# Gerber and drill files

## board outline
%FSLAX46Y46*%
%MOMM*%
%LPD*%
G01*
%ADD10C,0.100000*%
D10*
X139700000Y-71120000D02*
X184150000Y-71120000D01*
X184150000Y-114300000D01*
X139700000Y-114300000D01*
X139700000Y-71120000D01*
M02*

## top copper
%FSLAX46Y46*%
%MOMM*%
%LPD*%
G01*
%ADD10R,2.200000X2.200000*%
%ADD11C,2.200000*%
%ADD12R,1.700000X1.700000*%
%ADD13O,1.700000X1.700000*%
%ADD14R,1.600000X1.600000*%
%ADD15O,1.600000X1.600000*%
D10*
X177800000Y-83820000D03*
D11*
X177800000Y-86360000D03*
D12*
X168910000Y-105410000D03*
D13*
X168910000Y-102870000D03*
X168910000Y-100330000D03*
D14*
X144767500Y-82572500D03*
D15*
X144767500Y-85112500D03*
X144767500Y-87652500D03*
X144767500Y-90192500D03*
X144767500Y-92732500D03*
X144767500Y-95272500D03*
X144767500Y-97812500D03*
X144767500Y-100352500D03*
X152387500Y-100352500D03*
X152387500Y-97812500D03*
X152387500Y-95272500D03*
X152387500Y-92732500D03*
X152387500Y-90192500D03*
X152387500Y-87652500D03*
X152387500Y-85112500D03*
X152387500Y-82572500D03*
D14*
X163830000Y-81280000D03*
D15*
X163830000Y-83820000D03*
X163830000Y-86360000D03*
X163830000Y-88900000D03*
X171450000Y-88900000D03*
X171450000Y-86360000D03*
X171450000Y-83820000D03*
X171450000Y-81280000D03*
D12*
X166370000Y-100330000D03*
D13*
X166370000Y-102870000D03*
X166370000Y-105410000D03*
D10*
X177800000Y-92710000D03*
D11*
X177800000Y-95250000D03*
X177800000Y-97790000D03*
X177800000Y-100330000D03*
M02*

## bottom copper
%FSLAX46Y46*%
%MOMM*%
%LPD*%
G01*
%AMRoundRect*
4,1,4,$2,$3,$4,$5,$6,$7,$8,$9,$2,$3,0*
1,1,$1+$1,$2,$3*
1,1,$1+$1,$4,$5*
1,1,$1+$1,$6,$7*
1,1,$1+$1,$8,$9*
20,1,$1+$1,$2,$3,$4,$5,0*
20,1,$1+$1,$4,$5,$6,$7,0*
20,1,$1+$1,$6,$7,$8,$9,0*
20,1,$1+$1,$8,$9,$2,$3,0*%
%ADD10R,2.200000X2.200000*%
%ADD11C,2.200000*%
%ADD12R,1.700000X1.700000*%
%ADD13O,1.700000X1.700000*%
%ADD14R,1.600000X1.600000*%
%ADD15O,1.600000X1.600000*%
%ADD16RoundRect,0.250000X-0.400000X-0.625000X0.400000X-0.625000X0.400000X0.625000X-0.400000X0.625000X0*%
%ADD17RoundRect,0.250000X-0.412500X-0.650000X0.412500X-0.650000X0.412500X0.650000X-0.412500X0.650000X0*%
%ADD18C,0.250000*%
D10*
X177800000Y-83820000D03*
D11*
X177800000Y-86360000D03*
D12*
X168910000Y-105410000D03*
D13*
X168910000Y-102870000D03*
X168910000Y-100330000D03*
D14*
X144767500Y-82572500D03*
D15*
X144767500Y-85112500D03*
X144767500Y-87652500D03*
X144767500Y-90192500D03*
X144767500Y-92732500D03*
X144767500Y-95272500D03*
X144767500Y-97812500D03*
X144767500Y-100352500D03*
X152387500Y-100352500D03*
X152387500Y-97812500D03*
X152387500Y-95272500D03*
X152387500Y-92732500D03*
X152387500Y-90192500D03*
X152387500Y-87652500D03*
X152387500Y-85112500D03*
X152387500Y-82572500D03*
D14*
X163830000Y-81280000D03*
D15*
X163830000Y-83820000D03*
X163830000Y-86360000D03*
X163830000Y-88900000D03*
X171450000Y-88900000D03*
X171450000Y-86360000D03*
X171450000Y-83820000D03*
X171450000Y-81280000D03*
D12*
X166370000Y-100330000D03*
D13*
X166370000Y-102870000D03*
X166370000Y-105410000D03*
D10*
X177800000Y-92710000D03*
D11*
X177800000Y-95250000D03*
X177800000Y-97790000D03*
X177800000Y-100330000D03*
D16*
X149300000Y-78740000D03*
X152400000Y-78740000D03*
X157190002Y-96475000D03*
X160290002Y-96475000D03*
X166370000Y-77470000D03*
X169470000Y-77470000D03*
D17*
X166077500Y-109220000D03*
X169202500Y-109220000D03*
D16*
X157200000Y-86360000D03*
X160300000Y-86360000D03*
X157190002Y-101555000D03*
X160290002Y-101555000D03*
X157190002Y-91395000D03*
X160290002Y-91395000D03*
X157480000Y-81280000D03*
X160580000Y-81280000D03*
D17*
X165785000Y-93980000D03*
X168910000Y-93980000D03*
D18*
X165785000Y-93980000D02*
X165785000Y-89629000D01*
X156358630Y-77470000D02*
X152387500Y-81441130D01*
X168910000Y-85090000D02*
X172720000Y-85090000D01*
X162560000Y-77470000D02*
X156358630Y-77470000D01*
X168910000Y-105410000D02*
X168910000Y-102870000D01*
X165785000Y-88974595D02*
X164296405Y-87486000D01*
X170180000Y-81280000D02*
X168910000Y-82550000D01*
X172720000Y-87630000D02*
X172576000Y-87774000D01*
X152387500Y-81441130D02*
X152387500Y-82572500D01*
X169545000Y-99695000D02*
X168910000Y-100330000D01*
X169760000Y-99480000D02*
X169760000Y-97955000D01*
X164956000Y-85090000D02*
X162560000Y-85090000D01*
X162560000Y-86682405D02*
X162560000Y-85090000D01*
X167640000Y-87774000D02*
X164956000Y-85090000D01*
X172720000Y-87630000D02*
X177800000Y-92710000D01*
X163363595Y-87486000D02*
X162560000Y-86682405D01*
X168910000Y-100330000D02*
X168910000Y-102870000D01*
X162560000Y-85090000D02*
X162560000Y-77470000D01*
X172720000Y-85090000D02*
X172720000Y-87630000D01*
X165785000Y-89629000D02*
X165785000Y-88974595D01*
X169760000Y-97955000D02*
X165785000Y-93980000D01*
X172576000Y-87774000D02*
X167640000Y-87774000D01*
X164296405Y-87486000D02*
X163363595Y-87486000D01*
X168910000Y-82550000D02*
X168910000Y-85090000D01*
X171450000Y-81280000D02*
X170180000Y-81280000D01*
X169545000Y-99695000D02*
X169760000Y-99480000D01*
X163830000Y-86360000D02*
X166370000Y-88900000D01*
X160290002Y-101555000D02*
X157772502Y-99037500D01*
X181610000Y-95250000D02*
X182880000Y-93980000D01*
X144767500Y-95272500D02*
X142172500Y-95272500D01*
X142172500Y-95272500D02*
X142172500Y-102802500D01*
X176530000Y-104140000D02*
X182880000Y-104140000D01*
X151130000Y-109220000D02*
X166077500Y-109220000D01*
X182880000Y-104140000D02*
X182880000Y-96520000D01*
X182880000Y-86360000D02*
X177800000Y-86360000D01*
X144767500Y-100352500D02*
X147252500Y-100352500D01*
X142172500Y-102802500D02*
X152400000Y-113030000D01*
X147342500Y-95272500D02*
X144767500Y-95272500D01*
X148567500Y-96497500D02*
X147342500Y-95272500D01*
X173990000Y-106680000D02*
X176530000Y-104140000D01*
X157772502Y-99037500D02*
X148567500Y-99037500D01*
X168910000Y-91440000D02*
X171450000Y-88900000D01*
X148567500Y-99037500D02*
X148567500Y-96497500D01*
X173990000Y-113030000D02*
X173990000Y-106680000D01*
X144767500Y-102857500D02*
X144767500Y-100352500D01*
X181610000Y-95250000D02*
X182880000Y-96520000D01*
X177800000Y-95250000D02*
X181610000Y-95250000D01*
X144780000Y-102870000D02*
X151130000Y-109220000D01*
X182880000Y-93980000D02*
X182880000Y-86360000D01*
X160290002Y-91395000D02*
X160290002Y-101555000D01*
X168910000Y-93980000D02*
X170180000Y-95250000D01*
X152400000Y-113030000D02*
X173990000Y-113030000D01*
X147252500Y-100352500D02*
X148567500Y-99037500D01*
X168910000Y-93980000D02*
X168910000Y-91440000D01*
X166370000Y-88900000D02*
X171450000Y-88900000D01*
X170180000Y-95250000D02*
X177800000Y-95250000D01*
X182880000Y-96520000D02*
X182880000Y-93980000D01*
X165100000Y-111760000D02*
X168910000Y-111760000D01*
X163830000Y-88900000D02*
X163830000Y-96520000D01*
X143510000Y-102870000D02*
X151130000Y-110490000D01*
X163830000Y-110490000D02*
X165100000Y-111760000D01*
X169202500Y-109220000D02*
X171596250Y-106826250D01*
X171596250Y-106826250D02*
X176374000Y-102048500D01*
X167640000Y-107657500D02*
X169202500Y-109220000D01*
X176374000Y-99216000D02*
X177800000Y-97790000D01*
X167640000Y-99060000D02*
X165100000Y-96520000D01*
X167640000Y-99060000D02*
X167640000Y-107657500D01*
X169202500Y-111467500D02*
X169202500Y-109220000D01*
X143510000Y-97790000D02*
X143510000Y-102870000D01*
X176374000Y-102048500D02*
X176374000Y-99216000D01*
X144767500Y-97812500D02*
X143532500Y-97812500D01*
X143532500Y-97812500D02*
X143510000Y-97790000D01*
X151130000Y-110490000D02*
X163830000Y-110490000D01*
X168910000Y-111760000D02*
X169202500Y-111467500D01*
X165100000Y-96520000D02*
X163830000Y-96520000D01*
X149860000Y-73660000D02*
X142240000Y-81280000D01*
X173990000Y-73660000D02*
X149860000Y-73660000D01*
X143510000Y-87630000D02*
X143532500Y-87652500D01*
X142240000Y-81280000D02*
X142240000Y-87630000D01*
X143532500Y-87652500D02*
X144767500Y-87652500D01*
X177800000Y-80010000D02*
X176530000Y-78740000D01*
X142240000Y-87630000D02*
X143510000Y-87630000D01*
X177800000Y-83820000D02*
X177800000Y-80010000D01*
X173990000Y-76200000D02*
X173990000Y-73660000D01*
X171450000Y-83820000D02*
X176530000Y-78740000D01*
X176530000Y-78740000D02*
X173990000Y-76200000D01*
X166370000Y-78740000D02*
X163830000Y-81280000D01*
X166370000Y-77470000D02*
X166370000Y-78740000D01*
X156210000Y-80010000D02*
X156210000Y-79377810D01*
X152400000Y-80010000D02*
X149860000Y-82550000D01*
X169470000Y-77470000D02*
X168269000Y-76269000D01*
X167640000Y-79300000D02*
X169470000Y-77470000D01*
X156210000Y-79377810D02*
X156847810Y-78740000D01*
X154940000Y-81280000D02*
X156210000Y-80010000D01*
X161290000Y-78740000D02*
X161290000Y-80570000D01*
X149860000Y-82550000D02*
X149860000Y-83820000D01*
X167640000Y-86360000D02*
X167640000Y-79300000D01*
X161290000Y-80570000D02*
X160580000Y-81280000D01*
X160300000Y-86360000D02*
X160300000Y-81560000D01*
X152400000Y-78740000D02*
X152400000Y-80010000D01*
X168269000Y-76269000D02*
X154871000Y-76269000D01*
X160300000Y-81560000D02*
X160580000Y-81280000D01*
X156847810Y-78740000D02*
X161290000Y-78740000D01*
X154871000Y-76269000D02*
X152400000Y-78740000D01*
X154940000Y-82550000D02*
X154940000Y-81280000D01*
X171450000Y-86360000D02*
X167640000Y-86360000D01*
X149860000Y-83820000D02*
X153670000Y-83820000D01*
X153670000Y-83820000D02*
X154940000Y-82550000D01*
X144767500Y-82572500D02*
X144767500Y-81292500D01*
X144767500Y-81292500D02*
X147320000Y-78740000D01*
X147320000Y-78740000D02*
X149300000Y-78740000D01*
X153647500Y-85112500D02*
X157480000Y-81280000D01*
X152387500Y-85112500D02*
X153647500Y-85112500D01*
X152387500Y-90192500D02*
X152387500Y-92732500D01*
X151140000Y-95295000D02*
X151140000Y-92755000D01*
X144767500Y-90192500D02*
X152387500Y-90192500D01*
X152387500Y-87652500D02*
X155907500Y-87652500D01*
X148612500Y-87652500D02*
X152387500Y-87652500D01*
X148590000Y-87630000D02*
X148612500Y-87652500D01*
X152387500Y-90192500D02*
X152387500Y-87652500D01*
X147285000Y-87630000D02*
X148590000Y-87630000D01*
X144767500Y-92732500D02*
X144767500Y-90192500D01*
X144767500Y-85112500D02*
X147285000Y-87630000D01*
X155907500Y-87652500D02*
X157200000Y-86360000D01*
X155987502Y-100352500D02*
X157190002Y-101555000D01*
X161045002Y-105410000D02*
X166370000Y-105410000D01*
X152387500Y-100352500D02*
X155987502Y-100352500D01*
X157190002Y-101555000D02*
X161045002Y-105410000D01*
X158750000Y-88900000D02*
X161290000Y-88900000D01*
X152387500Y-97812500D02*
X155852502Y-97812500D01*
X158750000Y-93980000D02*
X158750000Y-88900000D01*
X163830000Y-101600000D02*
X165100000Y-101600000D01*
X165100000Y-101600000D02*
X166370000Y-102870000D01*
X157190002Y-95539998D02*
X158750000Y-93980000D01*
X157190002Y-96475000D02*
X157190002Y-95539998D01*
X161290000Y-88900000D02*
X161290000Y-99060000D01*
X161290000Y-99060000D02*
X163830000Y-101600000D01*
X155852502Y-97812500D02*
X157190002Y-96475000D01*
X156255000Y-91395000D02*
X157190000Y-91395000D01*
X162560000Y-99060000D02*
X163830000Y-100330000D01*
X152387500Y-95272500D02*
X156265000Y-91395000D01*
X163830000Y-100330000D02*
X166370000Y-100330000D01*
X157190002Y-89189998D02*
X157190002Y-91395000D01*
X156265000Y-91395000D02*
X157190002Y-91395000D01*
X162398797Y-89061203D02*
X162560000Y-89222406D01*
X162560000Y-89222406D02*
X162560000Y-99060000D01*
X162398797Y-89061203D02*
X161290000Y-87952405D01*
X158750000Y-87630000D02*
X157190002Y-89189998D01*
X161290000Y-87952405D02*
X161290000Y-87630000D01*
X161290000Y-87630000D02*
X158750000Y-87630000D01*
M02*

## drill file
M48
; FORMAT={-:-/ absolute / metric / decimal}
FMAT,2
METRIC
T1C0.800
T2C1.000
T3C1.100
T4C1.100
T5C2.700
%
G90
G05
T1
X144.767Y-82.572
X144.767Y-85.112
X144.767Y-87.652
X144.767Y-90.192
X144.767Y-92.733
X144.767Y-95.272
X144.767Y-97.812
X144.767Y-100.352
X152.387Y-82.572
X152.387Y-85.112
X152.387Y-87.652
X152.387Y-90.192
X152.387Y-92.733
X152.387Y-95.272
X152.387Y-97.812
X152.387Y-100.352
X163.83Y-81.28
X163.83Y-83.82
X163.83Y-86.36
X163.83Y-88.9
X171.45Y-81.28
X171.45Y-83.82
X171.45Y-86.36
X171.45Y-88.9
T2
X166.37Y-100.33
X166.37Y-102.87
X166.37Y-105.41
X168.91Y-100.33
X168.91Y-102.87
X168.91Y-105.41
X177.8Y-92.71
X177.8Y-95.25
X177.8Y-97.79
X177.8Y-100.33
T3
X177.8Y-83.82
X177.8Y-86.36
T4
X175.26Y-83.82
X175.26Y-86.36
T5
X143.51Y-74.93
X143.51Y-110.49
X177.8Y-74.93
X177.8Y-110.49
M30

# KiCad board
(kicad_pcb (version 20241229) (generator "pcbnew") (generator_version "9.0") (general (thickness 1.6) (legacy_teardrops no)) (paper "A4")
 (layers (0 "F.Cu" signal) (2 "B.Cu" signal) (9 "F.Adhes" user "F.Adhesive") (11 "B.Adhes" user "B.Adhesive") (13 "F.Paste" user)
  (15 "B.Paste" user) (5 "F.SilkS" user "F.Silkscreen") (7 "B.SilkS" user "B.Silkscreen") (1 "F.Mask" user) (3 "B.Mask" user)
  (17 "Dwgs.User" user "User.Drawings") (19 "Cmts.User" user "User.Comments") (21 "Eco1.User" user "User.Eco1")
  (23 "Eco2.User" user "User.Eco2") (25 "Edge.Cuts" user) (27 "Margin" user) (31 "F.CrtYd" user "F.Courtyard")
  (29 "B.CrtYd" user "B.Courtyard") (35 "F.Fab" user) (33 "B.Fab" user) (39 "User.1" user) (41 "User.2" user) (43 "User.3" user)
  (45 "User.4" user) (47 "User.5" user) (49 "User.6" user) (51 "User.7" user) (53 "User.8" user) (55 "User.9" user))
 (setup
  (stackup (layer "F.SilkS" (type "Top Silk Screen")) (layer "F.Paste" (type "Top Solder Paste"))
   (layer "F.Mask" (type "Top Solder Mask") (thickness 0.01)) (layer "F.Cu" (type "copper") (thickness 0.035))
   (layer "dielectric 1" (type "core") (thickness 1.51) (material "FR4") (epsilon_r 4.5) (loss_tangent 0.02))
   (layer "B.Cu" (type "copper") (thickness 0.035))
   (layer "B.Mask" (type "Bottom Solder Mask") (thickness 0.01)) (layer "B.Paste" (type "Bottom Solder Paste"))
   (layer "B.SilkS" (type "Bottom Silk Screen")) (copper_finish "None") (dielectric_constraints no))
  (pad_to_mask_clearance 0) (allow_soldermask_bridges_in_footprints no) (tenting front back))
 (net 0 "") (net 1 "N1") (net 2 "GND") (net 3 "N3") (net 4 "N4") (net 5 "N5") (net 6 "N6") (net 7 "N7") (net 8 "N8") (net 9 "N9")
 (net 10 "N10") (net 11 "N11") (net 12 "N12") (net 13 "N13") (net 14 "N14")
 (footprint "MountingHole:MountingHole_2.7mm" (layer "F.Cu") (at 177.8 74.93)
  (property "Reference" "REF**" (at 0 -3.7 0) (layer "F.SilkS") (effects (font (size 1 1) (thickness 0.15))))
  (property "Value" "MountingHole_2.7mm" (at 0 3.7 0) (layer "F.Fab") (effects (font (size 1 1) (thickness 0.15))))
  (pad "" np_thru_hole circle (at 0 0) (size 2.7 2.7) (drill 2.7) (layers "*.Cu" "*.Mask")))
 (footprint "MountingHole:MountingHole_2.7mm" (layer "F.Cu") (at 177.8 110.49)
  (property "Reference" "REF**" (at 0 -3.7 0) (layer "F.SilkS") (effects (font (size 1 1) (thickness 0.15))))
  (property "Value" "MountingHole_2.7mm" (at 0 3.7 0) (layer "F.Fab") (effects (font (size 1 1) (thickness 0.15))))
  (pad "" np_thru_hole circle (at 0 0) (size 2.7 2.7) (drill 2.7) (layers "*.Cu" "*.Mask")))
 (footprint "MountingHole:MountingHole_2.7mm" (layer "F.Cu") (at 143.51 110.49)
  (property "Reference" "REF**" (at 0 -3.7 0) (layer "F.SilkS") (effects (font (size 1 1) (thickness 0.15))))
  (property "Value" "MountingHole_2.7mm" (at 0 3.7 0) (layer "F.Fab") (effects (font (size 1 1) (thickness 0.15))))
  (pad "" np_thru_hole circle (at 0 0) (size 2.7 2.7) (drill 2.7) (layers "*.Cu" "*.Mask")))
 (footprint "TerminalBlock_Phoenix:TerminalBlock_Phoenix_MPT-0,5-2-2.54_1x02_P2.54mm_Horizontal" (layer "F.Cu") (at 177.8 83.82 -90)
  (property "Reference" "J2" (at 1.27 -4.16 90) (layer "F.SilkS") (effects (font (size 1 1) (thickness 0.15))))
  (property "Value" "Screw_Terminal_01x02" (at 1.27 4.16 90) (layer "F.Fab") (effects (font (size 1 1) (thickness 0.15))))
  (pad "" np_thru_hole circle (at 0 2.54 270) (size 1.1 1.1) (drill 1.1) (layers "*.Cu" "*.Mask"))
  (pad "" np_thru_hole circle (at 2.54 2.54 270) (size 1.1 1.1) (drill 1.1) (layers "*.Cu" "*.Mask"))
  (pad "1" thru_hole rect (at 0 0 270) (size 2.2 2.2) (drill 1.1) (layers "*.Cu" "*.Mask") (remove_unused_layers no) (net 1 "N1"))
  (pad "2" thru_hole circle (at 2.54 0 270) (size 2.2 2.2) (drill 1.1) (layers "*.Cu" "*.Mask") (remove_unused_layers no) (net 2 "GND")))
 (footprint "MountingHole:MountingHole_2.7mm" (layer "F.Cu") (at 143.51 74.93)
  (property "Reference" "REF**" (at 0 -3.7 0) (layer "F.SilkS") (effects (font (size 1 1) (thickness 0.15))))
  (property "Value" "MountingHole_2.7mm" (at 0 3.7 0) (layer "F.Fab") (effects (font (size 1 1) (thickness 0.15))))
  (pad "" np_thru_hole circle (at 0 0) (size 2.7 2.7) (drill 2.7) (layers "*.Cu" "*.Mask")))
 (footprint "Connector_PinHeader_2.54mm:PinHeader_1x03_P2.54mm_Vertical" (layer "F.Cu") (at 168.91 105.41 180)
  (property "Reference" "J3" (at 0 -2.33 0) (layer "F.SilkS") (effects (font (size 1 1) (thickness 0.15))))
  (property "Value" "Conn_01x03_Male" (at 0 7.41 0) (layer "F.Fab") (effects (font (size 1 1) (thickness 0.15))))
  (pad "1" thru_hole rect (at 0 0 180) (size 1.7 1.7) (drill 1) (layers "*.Cu" "*.Mask") (remove_unused_layers no) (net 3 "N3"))
  (pad "2" thru_hole oval (at 0 2.54 180) (size 1.7 1.7) (drill 1) (layers "*.Cu" "*.Mask") (remove_unused_layers no) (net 3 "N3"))
  (pad "3" thru_hole oval (at 0 5.08 180) (size 1.7 1.7) (drill 1) (layers "*.Cu" "*.Mask") (remove_unused_layers no) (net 3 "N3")))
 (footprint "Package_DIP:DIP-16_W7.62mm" (layer "F.Cu") (at 144.7675 82.5725)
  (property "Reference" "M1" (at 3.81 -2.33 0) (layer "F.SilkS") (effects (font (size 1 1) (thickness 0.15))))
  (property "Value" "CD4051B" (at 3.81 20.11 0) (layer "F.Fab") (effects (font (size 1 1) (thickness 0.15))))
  (pad "1" thru_hole rect (at 0 0) (size 1.6 1.6) (drill 0.8) (layers "*.Cu" "*.Mask") (remove_unused_layers no) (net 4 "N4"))
  (pad "2" thru_hole oval (at 0 2.54) (size 1.6 1.6) (drill 0.8) (layers "*.Cu" "*.Mask") (remove_unused_layers no) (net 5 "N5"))
  (pad "3" thru_hole oval (at 0 5.08) (size 1.6 1.6) (drill 0.8) (layers "*.Cu" "*.Mask") (remove_unused_layers no) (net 1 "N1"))
  (pad "4" thru_hole oval (at 0 7.62) (size 1.6 1.6) (drill 0.8) (layers "*.Cu" "*.Mask") (remove_unused_layers no) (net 5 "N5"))
  (pad "5" thru_hole oval (at 0 10.16) (size 1.6 1.6) (drill 0.8) (layers "*.Cu" "*.Mask") (remove_unused_layers no) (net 5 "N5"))
  (pad "6" thru_hole oval (at 0 12.7) (size 1.6 1.6) (drill 0.8) (layers "*.Cu" "*.Mask") (remove_unused_layers no) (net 2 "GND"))
  (pad "7" thru_hole oval (at 0 15.24) (size 1.6 1.6) (drill 0.8) (layers "*.Cu" "*.Mask") (remove_unused_layers no) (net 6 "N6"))
  (pad "8" thru_hole oval (at 0 17.78) (size 1.6 1.6) (drill 0.8) (layers "*.Cu" "*.Mask") (remove_unused_layers no) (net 2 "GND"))
  (pad "9" thru_hole oval (at 7.62 17.78) (size 1.6 1.6) (drill 0.8) (layers "*.Cu" "*.Mask") (remove_unused_layers no) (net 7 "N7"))
  (pad "10" thru_hole oval (at 7.62 15.24) (size 1.6 1.6) (drill 0.8) (layers "*.Cu" "*.Mask") (remove_unused_layers no) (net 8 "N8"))
  (pad "11" thru_hole oval (at 7.62 12.7) (size 1.6 1.6) (drill 0.8) (layers "*.Cu" "*.Mask") (remove_unused_layers no) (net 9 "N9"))
  (pad "12" thru_hole oval (at 7.62 10.16) (size 1.6 1.6) (drill 0.8) (layers "*.Cu" "*.Mask") (remove_unused_layers no) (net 5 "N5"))
  (pad "13" thru_hole oval (at 7.62 7.62) (size 1.6 1.6) (drill 0.8) (layers "*.Cu" "*.Mask") (remove_unused_layers no) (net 5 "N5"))
  (pad "14" thru_hole oval (at 7.62 5.08) (size 1.6 1.6) (drill 0.8) (layers "*.Cu" "*.Mask") (remove_unused_layers no) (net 5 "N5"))
  (pad "15" thru_hole oval (at 7.62 2.54) (size 1.6 1.6) (drill 0.8) (layers "*.Cu" "*.Mask") (remove_unused_layers no) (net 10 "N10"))
  (pad "16" thru_hole oval (at 7.62 0) (size 1.6 1.6) (drill 0.8) (layers "*.Cu" "*.Mask") (remove_unused_layers no) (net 3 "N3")))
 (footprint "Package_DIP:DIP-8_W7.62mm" (layer "F.Cu") (at 163.83 81.28)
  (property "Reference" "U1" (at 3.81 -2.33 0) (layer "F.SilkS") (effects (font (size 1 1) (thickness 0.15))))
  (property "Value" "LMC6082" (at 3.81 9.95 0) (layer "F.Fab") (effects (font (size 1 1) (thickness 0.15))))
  (pad "1" thru_hole rect (at 0 0) (size 1.6 1.6) (drill 0.8) (layers "*.Cu" "*.Mask") (remove_unused_layers no) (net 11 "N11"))
  (pad "2" thru_hole oval (at 0 2.54) (size 1.6 1.6) (drill 0.8) (layers "*.Cu" "*.Mask") (remove_unused_layers no) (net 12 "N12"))
  (pad "3" thru_hole oval (at 0 5.08) (size 1.6 1.6) (drill 0.8) (layers "*.Cu" "*.Mask") (remove_unused_layers no) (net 2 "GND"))
  (pad "4" thru_hole oval (at 0 7.62) (size 1.6 1.6) (drill 0.8) (layers "*.Cu" "*.Mask") (remove_unused_layers no) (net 6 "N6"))
  (pad "5" thru_hole oval (at 7.62 7.62) (size 1.6 1.6) (drill 0.8) (layers "*.Cu" "*.Mask") (remove_unused_layers no) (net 2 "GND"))
  (pad "6" thru_hole oval (at 7.62 5.08) (size 1.6 1.6) (drill 0.8) (layers "*.Cu" "*.Mask") (remove_unused_layers no) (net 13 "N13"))
  (pad "7" thru_hole oval (at 7.62 2.54) (size 1.6 1.6) (drill 0.8) (layers "*.Cu" "*.Mask") (remove_unused_layers no) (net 1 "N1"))
  (pad "8" thru_hole oval (at 7.62 0) (size 1.6 1.6) (drill 0.8) (layers "*.Cu" "*.Mask") (remove_unused_layers no) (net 3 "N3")))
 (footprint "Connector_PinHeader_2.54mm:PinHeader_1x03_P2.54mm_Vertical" (layer "F.Cu") (at 166.37 100.33)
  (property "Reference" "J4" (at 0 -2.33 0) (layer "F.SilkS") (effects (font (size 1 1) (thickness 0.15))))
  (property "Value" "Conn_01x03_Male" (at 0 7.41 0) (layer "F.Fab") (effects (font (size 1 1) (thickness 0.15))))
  (pad "1" thru_hole rect (at 0 0) (size 1.7 1.7) (drill 1) (layers "*.Cu" "*.Mask") (remove_unused_layers no) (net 9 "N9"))
  (pad "2" thru_hole oval (at 0 2.54) (size 1.7 1.7) (drill 1) (layers "*.Cu" "*.Mask") (remove_unused_layers no) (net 8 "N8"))
  (pad "3" thru_hole oval (at 0 5.08) (size 1.7 1.7) (drill 1) (layers "*.Cu" "*.Mask") (remove_unused_layers no) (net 7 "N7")))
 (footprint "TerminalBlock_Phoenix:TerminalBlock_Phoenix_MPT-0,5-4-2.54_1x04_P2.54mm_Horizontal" (layer "F.Cu") (at 177.8 92.71 -90)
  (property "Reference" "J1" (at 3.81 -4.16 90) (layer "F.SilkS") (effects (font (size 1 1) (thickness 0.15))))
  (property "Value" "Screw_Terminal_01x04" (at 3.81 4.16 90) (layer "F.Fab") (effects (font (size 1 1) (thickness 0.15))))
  (pad "1" thru_hole rect (at 0 0 270) (size 2.2 2.2) (drill 1) (layers "*.Cu" "*.Mask") (remove_unused_layers no) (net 3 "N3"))
  (pad "2" thru_hole circle (at 2.54 0 270) (size 2.2 2.2) (drill 1) (layers "*.Cu" "*.Mask") (remove_unused_layers no) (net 2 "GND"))
  (pad "3" thru_hole circle (at 5.08 0 270) (size 2.2 2.2) (drill 1) (layers "*.Cu" "*.Mask") (remove_unused_layers no) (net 6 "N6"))
  (pad "4" thru_hole circle (at 7.62 0 270) (size 2.2 2.2) (drill 1) (layers "*.Cu" "*.Mask") (remove_unused_layers no) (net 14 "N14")))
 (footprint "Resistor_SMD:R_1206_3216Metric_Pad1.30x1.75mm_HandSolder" (layer "B.Cu") (at 150.85 78.74)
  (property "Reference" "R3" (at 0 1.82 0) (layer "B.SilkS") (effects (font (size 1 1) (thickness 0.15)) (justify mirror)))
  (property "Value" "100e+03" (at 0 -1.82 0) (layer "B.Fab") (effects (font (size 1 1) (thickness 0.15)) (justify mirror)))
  (pad "1" smd roundrect (at -1.55 0) (size 1.3 1.75) (layers "B.Cu" "B.Mask" "B.Paste") (roundrect_rratio 0.1923076923) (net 4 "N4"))
  (pad "2" smd roundrect (at 1.55 0) (size 1.3 1.75) (layers "B.Cu" "B.Mask" "B.Paste") (roundrect_rratio 0.1923076923) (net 13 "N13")))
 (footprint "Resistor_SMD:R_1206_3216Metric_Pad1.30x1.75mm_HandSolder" (layer "B.Cu") (at 158.740002 96.475)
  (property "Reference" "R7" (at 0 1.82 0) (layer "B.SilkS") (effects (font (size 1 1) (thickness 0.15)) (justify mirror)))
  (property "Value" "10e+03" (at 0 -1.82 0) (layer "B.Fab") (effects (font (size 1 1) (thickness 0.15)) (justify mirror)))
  (pad "1" smd roundrect (at -1.55 0) (size 1.3 1.75) (layers "B.Cu" "B.Mask" "B.Paste") (roundrect_rratio 0.1923076923) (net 8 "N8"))
  (pad "2" smd roundrect (at 1.55 0) (size 1.3 1.75) (layers "B.Cu" "B.Mask" "B.Paste") (roundrect_rratio 0.1923076923) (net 2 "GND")))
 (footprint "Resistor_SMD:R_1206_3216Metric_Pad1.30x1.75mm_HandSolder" (layer "B.Cu") (at 167.92 77.47)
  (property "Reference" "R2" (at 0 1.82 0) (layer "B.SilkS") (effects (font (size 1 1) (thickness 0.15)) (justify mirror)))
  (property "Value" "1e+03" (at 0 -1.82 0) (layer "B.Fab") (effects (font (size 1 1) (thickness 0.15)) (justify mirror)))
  (pad "1" smd roundrect (at -1.55 0) (size 1.3 1.75) (layers "B.Cu" "B.Mask" "B.Paste") (roundrect_rratio 0.1923076923) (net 11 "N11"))
  (pad "2" smd roundrect (at 1.55 0) (size 1.3 1.75) (layers "B.Cu" "B.Mask" "B.Paste") (roundrect_rratio 0.1923076923) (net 13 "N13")))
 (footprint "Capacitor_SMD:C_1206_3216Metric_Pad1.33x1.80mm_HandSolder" (layer "B.Cu") (at 167.64 109.22)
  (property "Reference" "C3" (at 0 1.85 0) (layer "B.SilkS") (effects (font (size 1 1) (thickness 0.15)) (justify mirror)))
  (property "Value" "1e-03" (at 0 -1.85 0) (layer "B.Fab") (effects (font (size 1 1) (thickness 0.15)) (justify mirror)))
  (pad "1" smd roundrect (at -1.5625 0) (size 1.325 1.8) (layers "B.Cu" "B.Mask" "B.Paste") (roundrect_rratio 0.1886792453) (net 2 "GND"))
  (pad "2" smd roundrect (at 1.5625 0) (size 1.325 1.8) (layers "B.Cu" "B.Mask" "B.Paste") (roundrect_rratio 0.1886792453) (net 6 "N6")))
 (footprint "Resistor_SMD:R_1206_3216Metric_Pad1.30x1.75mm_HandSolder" (layer "B.Cu") (at 158.75 86.36)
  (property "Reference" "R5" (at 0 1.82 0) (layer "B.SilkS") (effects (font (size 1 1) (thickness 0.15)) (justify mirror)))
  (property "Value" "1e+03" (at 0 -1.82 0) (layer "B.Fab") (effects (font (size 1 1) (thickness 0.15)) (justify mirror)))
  (pad "1" smd roundrect (at -1.55 0) (size 1.3 1.75) (layers "B.Cu" "B.Mask" "B.Paste") (roundrect_rratio 0.1923076923) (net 5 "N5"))
  (pad "2" smd roundrect (at 1.55 0) (size 1.3 1.75) (layers "B.Cu" "B.Mask" "B.Paste") (roundrect_rratio 0.1923076923) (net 13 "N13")))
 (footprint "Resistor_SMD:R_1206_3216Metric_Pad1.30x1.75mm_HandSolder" (layer "B.Cu") (at 158.740002 101.555)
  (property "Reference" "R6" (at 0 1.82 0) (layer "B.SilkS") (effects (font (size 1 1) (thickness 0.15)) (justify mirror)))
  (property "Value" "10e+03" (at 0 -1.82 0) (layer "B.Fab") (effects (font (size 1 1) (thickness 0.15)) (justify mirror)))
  (pad "1" smd roundrect (at -1.55 0) (size 1.3 1.75) (layers "B.Cu" "B.Mask" "B.Paste") (roundrect_rratio 0.1923076923) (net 7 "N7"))
  (pad "2" smd roundrect (at 1.55 0) (size 1.3 1.75) (layers "B.Cu" "B.Mask" "B.Paste") (roundrect_rratio 0.1923076923) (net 2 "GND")))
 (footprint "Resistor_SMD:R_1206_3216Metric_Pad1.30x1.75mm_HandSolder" (layer "B.Cu") (at 158.740002 91.395)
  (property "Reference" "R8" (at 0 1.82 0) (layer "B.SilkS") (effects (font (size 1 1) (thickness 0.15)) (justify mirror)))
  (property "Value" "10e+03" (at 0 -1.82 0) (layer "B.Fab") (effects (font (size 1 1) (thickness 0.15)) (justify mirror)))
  (pad "1" smd roundrect (at -1.55 0) (size 1.3 1.75) (layers "B.Cu" "B.Mask" "B.Paste") (roundrect_rratio 0.1923076923) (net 9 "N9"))
  (pad "2" smd roundrect (at 1.55 0) (size 1.3 1.75) (layers "B.Cu" "B.Mask" "B.Paste") (roundrect_rratio 0.1923076923) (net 2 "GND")))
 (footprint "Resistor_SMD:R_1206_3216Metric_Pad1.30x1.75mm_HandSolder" (layer "B.Cu") (at 159.03 81.28)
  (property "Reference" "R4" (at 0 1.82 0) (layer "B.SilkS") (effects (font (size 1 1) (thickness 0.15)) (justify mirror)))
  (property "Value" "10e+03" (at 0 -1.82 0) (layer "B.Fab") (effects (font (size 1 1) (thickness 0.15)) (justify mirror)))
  (pad "1" smd roundrect (at -1.55 0) (size 1.3 1.75) (layers "B.Cu" "B.Mask" "B.Paste") (roundrect_rratio 0.1923076923) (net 10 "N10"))
  (pad "2" smd roundrect (at 1.55 0) (size 1.3 1.75) (layers "B.Cu" "B.Mask" "B.Paste") (roundrect_rratio 0.1923076923) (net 13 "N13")))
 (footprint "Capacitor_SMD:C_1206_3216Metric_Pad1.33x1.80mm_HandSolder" (layer "B.Cu") (at 167.3475 93.98)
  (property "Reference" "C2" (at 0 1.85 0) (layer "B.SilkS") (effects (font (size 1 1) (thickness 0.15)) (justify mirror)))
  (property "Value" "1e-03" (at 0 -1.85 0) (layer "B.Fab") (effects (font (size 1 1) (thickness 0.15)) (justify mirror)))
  (pad "1" smd roundrect (at -1.5625 0) (size 1.325 1.8) (layers "B.Cu" "B.Mask" "B.Paste") (roundrect_rratio 0.1886792453) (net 3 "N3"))
  (pad "2" smd roundrect (at 1.5625 0) (size 1.325 1.8) (layers "B.Cu" "B.Mask" "B.Paste") (roundrect_rratio 0.1886792453) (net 2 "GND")))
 (gr_rect (start 139.7 71.12) (end 184.15 114.3) (stroke (width 0.1) (type solid)) (fill no) (layer "Edge.Cuts"))
 (segment (start 165.785 93.98) (end 165.785 89.629) (width 0.25) (layer "B.Cu") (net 3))
 (segment (start 156.35863 77.47) (end 152.3875 81.44113) (width 0.25) (layer "B.Cu") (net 3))
 (segment (start 168.91 85.09) (end 172.72 85.09) (width 0.25) (layer "B.Cu") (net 3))
 (segment (start 162.56 77.47) (end 156.35863 77.47) (width 0.25) (layer "B.Cu") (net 3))
 (segment (start 168.91 105.41) (end 168.91 102.87) (width 0.25) (layer "B.Cu") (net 3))
 (segment (start 165.785 88.974595) (end 164.296405 87.486) (width 0.25) (layer "B.Cu") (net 3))
 (segment (start 170.18 81.28) (end 168.91 82.55) (width 0.25) (layer "B.Cu") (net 3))
 (segment (start 172.72 87.63) (end 172.576 87.774) (width 0.25) (layer "B.Cu") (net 3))
 (segment (start 152.3875 81.44113) (end 152.3875 82.5725) (width 0.25) (layer "B.Cu") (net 3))
 (segment (start 169.545 99.695) (end 168.91 100.33) (width 0.25) (layer "B.Cu") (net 3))
 (segment (start 169.76 99.48) (end 169.76 97.955) (width 0.25) (layer "B.Cu") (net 3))
 (segment (start 164.956 85.09) (end 162.56 85.09) (width 0.25) (layer "B.Cu") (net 3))
 (segment (start 162.56 86.682405) (end 162.56 85.09) (width 0.25) (layer "B.Cu") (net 3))
 (segment (start 167.64 87.774) (end 164.956 85.09) (width 0.25) (layer "B.Cu") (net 3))
 (segment (start 172.72 87.63) (end 177.8 92.71) (width 0.25) (layer "B.Cu") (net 3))
 (segment (start 163.363595 87.486) (end 162.56 86.682405) (width 0.25) (layer "B.Cu") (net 3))
 (segment (start 168.91 100.33) (end 168.91 102.87) (width 0.25) (layer "B.Cu") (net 3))
 (segment (start 162.56 85.09) (end 162.56 77.47) (width 0.25) (layer "B.Cu") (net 3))
 (segment (start 172.72 85.09) (end 172.72 87.63) (width 0.25) (layer "B.Cu") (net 3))
 (segment (start 165.785 89.629) (end 165.785 88.974595) (width 0.25) (layer "B.Cu") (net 3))
 (segment (start 169.76 97.955) (end 165.785 93.98) (width 0.25) (layer "B.Cu") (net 3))
 (segment (start 172.576 87.774) (end 167.64 87.774) (width 0.25) (layer "B.Cu") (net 3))
 (segment (start 164.296405 87.486) (end 163.363595 87.486) (width 0.25) (layer "B.Cu") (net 3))
 (segment (start 168.91 82.55) (end 168.91 85.09) (width 0.25) (layer "B.Cu") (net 3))
 (segment (start 171.45 81.28) (end 170.18 81.28) (width 0.25) (layer "B.Cu") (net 3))
 (segment (start 169.545 99.695) (end 169.76 99.48) (width 0.25) (layer "B.Cu") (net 3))
 (segment (start 163.83 86.36) (end 166.37 88.9) (width 0.25) (layer "B.Cu") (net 2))
 (segment (start 160.290002 101.555) (end 157.772502 99.0375) (width 0.25) (layer "B.Cu") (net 2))
 (segment (start 181.61 95.25) (end 182.88 93.98) (width 0.25) (layer "B.Cu") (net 2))
 (segment (start 144.7675 95.2725) (end 142.1725 95.2725) (width 0.25) (layer "B.Cu") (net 2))
 (segment (start 142.1725 95.2725) (end 142.1725 102.8025) (width 0.25) (layer "B.Cu") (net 2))
 (segment (start 176.53 104.14) (end 182.88 104.14) (width 0.25) (layer "B.Cu") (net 2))
 (segment (start 151.13 109.22) (end 166.0775 109.22) (width 0.25) (layer "B.Cu") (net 2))
 (segment (start 182.88 104.14) (end 182.88 96.52) (width 0.25) (layer "B.Cu") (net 2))
 (segment (start 182.88 86.36) (end 177.8 86.36) (width 0.25) (layer "B.Cu") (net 2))
 (segment (start 144.7675 100.3525) (end 147.2525 100.3525) (width 0.25) (layer "B.Cu") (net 2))
 (segment (start 142.1725 102.8025) (end 152.4 113.03) (width 0.25) (layer "B.Cu") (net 2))
 (segment (start 147.3425 95.2725) (end 144.7675 95.2725) (width 0.25) (layer "B.Cu") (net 2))
 (segment (start 148.5675 96.4975) (end 147.3425 95.2725) (width 0.25) (layer "B.Cu") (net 2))
 (segment (start 173.99 106.68) (end 176.53 104.14) (width 0.25) (layer "B.Cu") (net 2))
 (segment (start 157.772502 99.0375) (end 148.5675 99.0375) (width 0.25) (layer "B.Cu") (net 2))
 (segment (start 168.91 91.44) (end 171.45 88.9) (width 0.25) (layer "B.Cu") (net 2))
 (segment (start 148.5675 99.0375) (end 148.5675 96.4975) (width 0.25) (layer "B.Cu") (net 2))
 (segment (start 173.99 113.03) (end 173.99 106.68) (width 0.25) (layer "B.Cu") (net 2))
 (segment (start 144.7675 102.8575) (end 144.7675 100.3525) (width 0.25) (layer "B.Cu") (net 2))
 (segment (start 181.61 95.25) (end 182.88 96.52) (width 0.25) (layer "B.Cu") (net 2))
 (segment (start 177.8 95.25) (end 181.61 95.25) (width 0.25) (layer "B.Cu") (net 2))
 (segment (start 144.78 102.87) (end 151.13 109.22) (width 0.25) (layer "B.Cu") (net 2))
 (segment (start 182.88 93.98) (end 182.88 86.36) (width 0.25) (layer "B.Cu") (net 2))
 (segment (start 160.290002 91.395) (end 160.290002 101.555) (width 0.25) (layer "B.Cu") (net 2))
 (segment (start 168.91 93.98) (end 170.18 95.25) (width 0.25) (layer "B.Cu") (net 2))
 (segment (start 152.4 113.03) (end 173.99 113.03) (width 0.25) (layer "B.Cu") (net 2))
 (segment (start 147.2525 100.3525) (end 148.5675 99.0375) (width 0.25) (layer "B.Cu") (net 2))
 (segment (start 168.91 93.98) (end 168.91 91.44) (width 0.25) (layer "B.Cu") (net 2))
 (segment (start 166.37 88.9) (end 171.45 88.9) (width 0.25) (layer "B.Cu") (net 2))
 (segment (start 170.18 95.25) (end 177.8 95.25) (width 0.25) (layer "B.Cu") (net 2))
 (segment (start 182.88 96.52) (end 182.88 93.98) (width 0.25) (layer "B.Cu") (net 2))
 (segment (start 165.1 111.76) (end 168.91 111.76) (width 0.25) (layer "B.Cu") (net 6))
 (segment (start 163.83 88.9) (end 163.83 96.52) (width 0.25) (layer "B.Cu") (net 6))
 (segment (start 143.51 102.87) (end 151.13 110.49) (width 0.25) (layer "B.Cu") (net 6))
 (segment (start 163.83 110.49) (end 165.1 111.76) (width 0.25) (layer "B.Cu") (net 6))
 (segment (start 169.2025 109.22) (end 171.59625 106.82625) (width 0.25) (layer "B.Cu") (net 6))
 (segment (start 171.59625 106.82625) (end 176.374 102.0485) (width 0.25) (layer "B.Cu") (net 6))
 (segment (start 167.64 107.6575) (end 169.2025 109.22) (width 0.25) (layer "B.Cu") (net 6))
 (segment (start 176.374 99.216) (end 177.8 97.79) (width 0.25) (layer "B.Cu") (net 6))
 (segment (start 167.64 99.06) (end 165.1 96.52) (width 0.25) (layer "B.Cu") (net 6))
 (segment (start 167.64 99.06) (end 167.64 107.6575) (width 0.25) (layer "B.Cu") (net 6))
 (segment (start 169.2025 111.4675) (end 169.2025 109.22) (width 0.25) (layer "B.Cu") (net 6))
 (segment (start 143.51 97.79) (end 143.51 102.87) (width 0.25) (layer "B.Cu") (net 6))
 (segment (start 176.374 102.0485) (end 176.374 99.216) (width 0.25) (layer "B.Cu") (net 6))
 (segment (start 144.7675 97.8125) (end 143.5325 97.8125) (width 0.25) (layer "B.Cu") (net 6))
 (segment (start 143.5325 97.8125) (end 143.51 97.79) (width 0.25) (layer "B.Cu") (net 6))
 (segment (start 151.13 110.49) (end 163.83 110.49) (width 0.25) (layer "B.Cu") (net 6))
 (segment (start 168.91 111.76) (end 169.2025 111.4675) (width 0.25) (layer "B.Cu") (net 6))
 (segment (start 165.1 96.52) (end 163.83 96.52) (width 0.25) (layer "B.Cu") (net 6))
 (segment (start 149.86 73.66) (end 142.24 81.28) (width 0.25) (layer "B.Cu") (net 1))
 (segment (start 173.99 73.66) (end 149.86 73.66) (width 0.25) (layer "B.Cu") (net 1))
 (segment (start 143.51 87.63) (end 143.5325 87.6525) (width 0.25) (layer "B.Cu") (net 1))
 (segment (start 142.24 81.28) (end 142.24 87.63) (width 0.25) (layer "B.Cu") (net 1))
 (segment (start 143.5325 87.6525) (end 144.7675 87.6525) (width 0.25) (layer "B.Cu") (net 1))
 (segment (start 177.8 80.01) (end 176.53 78.74) (width 0.25) (layer "B.Cu") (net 1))
 (segment (start 142.24 87.63) (end 143.51 87.63) (width 0.25) (layer "B.Cu") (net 1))
 (segment (start 177.8 83.82) (end 177.8 80.01) (width 0.25) (layer "B.Cu") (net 1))
 (segment (start 173.99 76.2) (end 173.99 73.66) (width 0.25) (layer "B.Cu") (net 1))
 (segment (start 171.45 83.82) (end 176.53 78.74) (width 0.25) (layer "B.Cu") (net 1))
 (segment (start 176.53 78.74) (end 173.99 76.2) (width 0.25) (layer "B.Cu") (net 1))
 (segment (start 166.37 78.74) (end 163.83 81.28) (width 0.25) (layer "B.Cu") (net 11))
 (segment (start 166.37 77.47) (end 166.37 78.74) (width 0.25) (layer "B.Cu") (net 11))
 (segment (start 156.21 80.01) (end 156.21 79.37781) (width 0.25) (layer "B.Cu") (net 13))
 (segment (start 152.4 80.01) (end 149.86 82.55) (width 0.25) (layer "B.Cu") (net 13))
 (segment (start 169.47 77.47) (end 168.269 76.269) (width 0.25) (layer "B.Cu") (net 13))
 (segment (start 167.64 79.3) (end 169.47 77.47) (width 0.25) (layer "B.Cu") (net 13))
 (segment (start 156.21 79.37781) (end 156.84781 78.74) (width 0.25) (layer "B.Cu") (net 13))
 (segment (start 154.94 81.28) (end 156.21 80.01) (width 0.25) (layer "B.Cu") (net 13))
 (segment (start 161.29 78.74) (end 161.29 80.57) (width 0.25) (layer "B.Cu") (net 13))
 (segment (start 149.86 82.55) (end 149.86 83.82) (width 0.25) (layer "B.Cu") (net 13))
 (segment (start 167.64 86.36) (end 167.64 79.3) (width 0.25) (layer "B.Cu") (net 13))
 (segment (start 161.29 80.57) (end 160.58 81.28) (width 0.25) (layer "B.Cu") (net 13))
 (segment (start 160.3 86.36) (end 160.3 81.56) (width 0.25) (layer "B.Cu") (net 13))
 (segment (start 152.4 78.74) (end 152.4 80.01) (width 0.25) (layer "B.Cu") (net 13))
 (segment (start 168.269 76.269) (end 154.871 76.269) (width 0.25) (layer "B.Cu") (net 13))
 (segment (start 160.3 81.56) (end 160.58 81.28) (width 0.25) (layer "B.Cu") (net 13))
 (segment (start 156.84781 78.74) (end 161.29 78.74) (width 0.25) (layer "B.Cu") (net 13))
 (segment (start 154.871 76.269) (end 152.4 78.74) (width 0.25) (layer "B.Cu") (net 13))
 (segment (start 154.94 82.55) (end 154.94 81.28) (width 0.25) (layer "B.Cu") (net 13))
 (segment (start 171.45 86.36) (end 167.64 86.36) (width 0.25) (layer "B.Cu") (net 13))
 (segment (start 149.86 83.82) (end 153.67 83.82) (width 0.25) (layer "B.Cu") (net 13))
 (segment (start 153.67 83.82) (end 154.94 82.55) (width 0.25) (layer "B.Cu") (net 13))
 (segment (start 144.7675 82.5725) (end 144.7675 81.2925) (width 0.25) (layer "B.Cu") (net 4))
 (segment (start 144.7675 81.2925) (end 147.32 78.74) (width 0.25) (layer "B.Cu") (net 4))
 (segment (start 147.32 78.74) (end 149.3 78.74) (width 0.25) (layer "B.Cu") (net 4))
 (segment (start 153.6475 85.1125) (end 157.48 81.28) (width 0.25) (layer "B.Cu") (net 10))
 (segment (start 152.3875 85.1125) (end 153.6475 85.1125) (width 0.25) (layer "B.Cu") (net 10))
 (segment (start 152.3875 90.1925) (end 152.3875 92.7325) (width 0.25) (layer "B.Cu") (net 5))
 (segment (start 151.14 95.295) (end 151.14 92.755) (width 0.25) (layer "B.Cu") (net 5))
 (segment (start 144.7675 90.1925) (end 152.3875 90.1925) (width 0.25) (layer "B.Cu") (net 5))
 (segment (start 152.3875 87.6525) (end 155.9075 87.6525) (width 0.25) (layer "B.Cu") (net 5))
 (segment (start 148.6125 87.6525) (end 152.3875 87.6525) (width 0.25) (layer "B.Cu") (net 5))
 (segment (start 148.59 87.63) (end 148.6125 87.6525) (width 0.25) (layer "B.Cu") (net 5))
 (segment (start 152.3875 90.1925) (end 152.3875 87.6525) (width 0.25) (layer "B.Cu") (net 5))
 (segment (start 147.285 87.63) (end 148.59 87.63) (width 0.25) (layer "B.Cu") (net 5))
 (segment (start 144.7675 92.7325) (end 144.7675 90.1925) (width 0.25) (layer "B.Cu") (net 5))
 (segment (start 144.7675 85.1125) (end 147.285 87.63) (width 0.25) (layer "B.Cu") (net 5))
 (segment (start 155.9075 87.6525) (end 157.2 86.36) (width 0.25) (layer "B.Cu") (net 5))
 (segment (start 155.987502 100.3525) (end 157.190002 101.555) (width 0.25) (layer "B.Cu") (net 7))
 (segment (start 161.045002 105.41) (end 166.37 105.41) (width 0.25) (layer "B.Cu") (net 7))
 (segment (start 152.3875 100.3525) (end 155.987502 100.3525) (width 0.25) (layer "B.Cu") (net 7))
 (segment (start 157.190002 101.555) (end 161.045002 105.41) (width 0.25) (layer "B.Cu") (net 7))
 (segment (start 158.75 88.9) (end 161.29 88.9) (width 0.25) (layer "B.Cu") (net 8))
 (segment (start 152.3875 97.8125) (end 155.852502 97.8125) (width 0.25) (layer "B.Cu") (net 8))
 (segment (start 158.75 93.98) (end 158.75 88.9) (width 0.25) (layer "B.Cu") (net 8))
 (segment (start 163.83 101.6) (end 165.1 101.6) (width 0.25) (layer "B.Cu") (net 8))
 (segment (start 165.1 101.6) (end 166.37 102.87) (width 0.25) (layer "B.Cu") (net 8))
 (segment (start 157.190002 95.539998) (end 158.75 93.98) (width 0.25) (layer "B.Cu") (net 8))
 (segment (start 157.190002 96.475) (end 157.190002 95.539998) (width 0.25) (layer "B.Cu") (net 8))
 (segment (start 161.29 88.9) (end 161.29 99.06) (width 0.25) (layer "B.Cu") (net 8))
 (segment (start 161.29 99.06) (end 163.83 101.6) (width 0.25) (layer "B.Cu") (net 8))
 (segment (start 155.852502 97.8125) (end 157.190002 96.475) (width 0.25) (layer "B.Cu") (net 8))
 (segment (start 156.255 91.395) (end 157.19 91.395) (width 0.25) (layer "B.Cu") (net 9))
 (segment (start 162.56 99.06) (end 163.83 100.33) (width 0.25) (layer "B.Cu") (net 9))
 (segment (start 152.3875 95.2725) (end 156.265 91.395) (width 0.25) (layer "B.Cu") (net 9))
 (segment (start 163.83 100.33) (end 166.37 100.33) (width 0.25) (layer "B.Cu") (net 9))
 (segment (start 157.190002 89.189998) (end 157.190002 91.395) (width 0.25) (layer "B.Cu") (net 9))
 (segment (start 156.265 91.395) (end 157.190002 91.395) (width 0.25) (layer "B.Cu") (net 9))
 (segment (start 162.398797 89.061203) (end 162.56 89.222406) (width 0.25) (layer "B.Cu") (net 9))
 (segment (start 162.56 89.222406) (end 162.56 99.06) (width 0.25) (layer "B.Cu") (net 9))
 (segment (start 162.398797 89.061203) (end 161.29 87.952405) (width 0.25) (layer "B.Cu") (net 9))
 (segment (start 158.75 87.63) (end 157.190002 89.189998) (width 0.25) (layer "B.Cu") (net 9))
 (segment (start 161.29 87.952405) (end 161.29 87.63) (width 0.25) (layer "B.Cu") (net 9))
 (segment (start 161.29 87.63) (end 158.75 87.63) (width 0.25) (layer "B.Cu") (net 9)))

